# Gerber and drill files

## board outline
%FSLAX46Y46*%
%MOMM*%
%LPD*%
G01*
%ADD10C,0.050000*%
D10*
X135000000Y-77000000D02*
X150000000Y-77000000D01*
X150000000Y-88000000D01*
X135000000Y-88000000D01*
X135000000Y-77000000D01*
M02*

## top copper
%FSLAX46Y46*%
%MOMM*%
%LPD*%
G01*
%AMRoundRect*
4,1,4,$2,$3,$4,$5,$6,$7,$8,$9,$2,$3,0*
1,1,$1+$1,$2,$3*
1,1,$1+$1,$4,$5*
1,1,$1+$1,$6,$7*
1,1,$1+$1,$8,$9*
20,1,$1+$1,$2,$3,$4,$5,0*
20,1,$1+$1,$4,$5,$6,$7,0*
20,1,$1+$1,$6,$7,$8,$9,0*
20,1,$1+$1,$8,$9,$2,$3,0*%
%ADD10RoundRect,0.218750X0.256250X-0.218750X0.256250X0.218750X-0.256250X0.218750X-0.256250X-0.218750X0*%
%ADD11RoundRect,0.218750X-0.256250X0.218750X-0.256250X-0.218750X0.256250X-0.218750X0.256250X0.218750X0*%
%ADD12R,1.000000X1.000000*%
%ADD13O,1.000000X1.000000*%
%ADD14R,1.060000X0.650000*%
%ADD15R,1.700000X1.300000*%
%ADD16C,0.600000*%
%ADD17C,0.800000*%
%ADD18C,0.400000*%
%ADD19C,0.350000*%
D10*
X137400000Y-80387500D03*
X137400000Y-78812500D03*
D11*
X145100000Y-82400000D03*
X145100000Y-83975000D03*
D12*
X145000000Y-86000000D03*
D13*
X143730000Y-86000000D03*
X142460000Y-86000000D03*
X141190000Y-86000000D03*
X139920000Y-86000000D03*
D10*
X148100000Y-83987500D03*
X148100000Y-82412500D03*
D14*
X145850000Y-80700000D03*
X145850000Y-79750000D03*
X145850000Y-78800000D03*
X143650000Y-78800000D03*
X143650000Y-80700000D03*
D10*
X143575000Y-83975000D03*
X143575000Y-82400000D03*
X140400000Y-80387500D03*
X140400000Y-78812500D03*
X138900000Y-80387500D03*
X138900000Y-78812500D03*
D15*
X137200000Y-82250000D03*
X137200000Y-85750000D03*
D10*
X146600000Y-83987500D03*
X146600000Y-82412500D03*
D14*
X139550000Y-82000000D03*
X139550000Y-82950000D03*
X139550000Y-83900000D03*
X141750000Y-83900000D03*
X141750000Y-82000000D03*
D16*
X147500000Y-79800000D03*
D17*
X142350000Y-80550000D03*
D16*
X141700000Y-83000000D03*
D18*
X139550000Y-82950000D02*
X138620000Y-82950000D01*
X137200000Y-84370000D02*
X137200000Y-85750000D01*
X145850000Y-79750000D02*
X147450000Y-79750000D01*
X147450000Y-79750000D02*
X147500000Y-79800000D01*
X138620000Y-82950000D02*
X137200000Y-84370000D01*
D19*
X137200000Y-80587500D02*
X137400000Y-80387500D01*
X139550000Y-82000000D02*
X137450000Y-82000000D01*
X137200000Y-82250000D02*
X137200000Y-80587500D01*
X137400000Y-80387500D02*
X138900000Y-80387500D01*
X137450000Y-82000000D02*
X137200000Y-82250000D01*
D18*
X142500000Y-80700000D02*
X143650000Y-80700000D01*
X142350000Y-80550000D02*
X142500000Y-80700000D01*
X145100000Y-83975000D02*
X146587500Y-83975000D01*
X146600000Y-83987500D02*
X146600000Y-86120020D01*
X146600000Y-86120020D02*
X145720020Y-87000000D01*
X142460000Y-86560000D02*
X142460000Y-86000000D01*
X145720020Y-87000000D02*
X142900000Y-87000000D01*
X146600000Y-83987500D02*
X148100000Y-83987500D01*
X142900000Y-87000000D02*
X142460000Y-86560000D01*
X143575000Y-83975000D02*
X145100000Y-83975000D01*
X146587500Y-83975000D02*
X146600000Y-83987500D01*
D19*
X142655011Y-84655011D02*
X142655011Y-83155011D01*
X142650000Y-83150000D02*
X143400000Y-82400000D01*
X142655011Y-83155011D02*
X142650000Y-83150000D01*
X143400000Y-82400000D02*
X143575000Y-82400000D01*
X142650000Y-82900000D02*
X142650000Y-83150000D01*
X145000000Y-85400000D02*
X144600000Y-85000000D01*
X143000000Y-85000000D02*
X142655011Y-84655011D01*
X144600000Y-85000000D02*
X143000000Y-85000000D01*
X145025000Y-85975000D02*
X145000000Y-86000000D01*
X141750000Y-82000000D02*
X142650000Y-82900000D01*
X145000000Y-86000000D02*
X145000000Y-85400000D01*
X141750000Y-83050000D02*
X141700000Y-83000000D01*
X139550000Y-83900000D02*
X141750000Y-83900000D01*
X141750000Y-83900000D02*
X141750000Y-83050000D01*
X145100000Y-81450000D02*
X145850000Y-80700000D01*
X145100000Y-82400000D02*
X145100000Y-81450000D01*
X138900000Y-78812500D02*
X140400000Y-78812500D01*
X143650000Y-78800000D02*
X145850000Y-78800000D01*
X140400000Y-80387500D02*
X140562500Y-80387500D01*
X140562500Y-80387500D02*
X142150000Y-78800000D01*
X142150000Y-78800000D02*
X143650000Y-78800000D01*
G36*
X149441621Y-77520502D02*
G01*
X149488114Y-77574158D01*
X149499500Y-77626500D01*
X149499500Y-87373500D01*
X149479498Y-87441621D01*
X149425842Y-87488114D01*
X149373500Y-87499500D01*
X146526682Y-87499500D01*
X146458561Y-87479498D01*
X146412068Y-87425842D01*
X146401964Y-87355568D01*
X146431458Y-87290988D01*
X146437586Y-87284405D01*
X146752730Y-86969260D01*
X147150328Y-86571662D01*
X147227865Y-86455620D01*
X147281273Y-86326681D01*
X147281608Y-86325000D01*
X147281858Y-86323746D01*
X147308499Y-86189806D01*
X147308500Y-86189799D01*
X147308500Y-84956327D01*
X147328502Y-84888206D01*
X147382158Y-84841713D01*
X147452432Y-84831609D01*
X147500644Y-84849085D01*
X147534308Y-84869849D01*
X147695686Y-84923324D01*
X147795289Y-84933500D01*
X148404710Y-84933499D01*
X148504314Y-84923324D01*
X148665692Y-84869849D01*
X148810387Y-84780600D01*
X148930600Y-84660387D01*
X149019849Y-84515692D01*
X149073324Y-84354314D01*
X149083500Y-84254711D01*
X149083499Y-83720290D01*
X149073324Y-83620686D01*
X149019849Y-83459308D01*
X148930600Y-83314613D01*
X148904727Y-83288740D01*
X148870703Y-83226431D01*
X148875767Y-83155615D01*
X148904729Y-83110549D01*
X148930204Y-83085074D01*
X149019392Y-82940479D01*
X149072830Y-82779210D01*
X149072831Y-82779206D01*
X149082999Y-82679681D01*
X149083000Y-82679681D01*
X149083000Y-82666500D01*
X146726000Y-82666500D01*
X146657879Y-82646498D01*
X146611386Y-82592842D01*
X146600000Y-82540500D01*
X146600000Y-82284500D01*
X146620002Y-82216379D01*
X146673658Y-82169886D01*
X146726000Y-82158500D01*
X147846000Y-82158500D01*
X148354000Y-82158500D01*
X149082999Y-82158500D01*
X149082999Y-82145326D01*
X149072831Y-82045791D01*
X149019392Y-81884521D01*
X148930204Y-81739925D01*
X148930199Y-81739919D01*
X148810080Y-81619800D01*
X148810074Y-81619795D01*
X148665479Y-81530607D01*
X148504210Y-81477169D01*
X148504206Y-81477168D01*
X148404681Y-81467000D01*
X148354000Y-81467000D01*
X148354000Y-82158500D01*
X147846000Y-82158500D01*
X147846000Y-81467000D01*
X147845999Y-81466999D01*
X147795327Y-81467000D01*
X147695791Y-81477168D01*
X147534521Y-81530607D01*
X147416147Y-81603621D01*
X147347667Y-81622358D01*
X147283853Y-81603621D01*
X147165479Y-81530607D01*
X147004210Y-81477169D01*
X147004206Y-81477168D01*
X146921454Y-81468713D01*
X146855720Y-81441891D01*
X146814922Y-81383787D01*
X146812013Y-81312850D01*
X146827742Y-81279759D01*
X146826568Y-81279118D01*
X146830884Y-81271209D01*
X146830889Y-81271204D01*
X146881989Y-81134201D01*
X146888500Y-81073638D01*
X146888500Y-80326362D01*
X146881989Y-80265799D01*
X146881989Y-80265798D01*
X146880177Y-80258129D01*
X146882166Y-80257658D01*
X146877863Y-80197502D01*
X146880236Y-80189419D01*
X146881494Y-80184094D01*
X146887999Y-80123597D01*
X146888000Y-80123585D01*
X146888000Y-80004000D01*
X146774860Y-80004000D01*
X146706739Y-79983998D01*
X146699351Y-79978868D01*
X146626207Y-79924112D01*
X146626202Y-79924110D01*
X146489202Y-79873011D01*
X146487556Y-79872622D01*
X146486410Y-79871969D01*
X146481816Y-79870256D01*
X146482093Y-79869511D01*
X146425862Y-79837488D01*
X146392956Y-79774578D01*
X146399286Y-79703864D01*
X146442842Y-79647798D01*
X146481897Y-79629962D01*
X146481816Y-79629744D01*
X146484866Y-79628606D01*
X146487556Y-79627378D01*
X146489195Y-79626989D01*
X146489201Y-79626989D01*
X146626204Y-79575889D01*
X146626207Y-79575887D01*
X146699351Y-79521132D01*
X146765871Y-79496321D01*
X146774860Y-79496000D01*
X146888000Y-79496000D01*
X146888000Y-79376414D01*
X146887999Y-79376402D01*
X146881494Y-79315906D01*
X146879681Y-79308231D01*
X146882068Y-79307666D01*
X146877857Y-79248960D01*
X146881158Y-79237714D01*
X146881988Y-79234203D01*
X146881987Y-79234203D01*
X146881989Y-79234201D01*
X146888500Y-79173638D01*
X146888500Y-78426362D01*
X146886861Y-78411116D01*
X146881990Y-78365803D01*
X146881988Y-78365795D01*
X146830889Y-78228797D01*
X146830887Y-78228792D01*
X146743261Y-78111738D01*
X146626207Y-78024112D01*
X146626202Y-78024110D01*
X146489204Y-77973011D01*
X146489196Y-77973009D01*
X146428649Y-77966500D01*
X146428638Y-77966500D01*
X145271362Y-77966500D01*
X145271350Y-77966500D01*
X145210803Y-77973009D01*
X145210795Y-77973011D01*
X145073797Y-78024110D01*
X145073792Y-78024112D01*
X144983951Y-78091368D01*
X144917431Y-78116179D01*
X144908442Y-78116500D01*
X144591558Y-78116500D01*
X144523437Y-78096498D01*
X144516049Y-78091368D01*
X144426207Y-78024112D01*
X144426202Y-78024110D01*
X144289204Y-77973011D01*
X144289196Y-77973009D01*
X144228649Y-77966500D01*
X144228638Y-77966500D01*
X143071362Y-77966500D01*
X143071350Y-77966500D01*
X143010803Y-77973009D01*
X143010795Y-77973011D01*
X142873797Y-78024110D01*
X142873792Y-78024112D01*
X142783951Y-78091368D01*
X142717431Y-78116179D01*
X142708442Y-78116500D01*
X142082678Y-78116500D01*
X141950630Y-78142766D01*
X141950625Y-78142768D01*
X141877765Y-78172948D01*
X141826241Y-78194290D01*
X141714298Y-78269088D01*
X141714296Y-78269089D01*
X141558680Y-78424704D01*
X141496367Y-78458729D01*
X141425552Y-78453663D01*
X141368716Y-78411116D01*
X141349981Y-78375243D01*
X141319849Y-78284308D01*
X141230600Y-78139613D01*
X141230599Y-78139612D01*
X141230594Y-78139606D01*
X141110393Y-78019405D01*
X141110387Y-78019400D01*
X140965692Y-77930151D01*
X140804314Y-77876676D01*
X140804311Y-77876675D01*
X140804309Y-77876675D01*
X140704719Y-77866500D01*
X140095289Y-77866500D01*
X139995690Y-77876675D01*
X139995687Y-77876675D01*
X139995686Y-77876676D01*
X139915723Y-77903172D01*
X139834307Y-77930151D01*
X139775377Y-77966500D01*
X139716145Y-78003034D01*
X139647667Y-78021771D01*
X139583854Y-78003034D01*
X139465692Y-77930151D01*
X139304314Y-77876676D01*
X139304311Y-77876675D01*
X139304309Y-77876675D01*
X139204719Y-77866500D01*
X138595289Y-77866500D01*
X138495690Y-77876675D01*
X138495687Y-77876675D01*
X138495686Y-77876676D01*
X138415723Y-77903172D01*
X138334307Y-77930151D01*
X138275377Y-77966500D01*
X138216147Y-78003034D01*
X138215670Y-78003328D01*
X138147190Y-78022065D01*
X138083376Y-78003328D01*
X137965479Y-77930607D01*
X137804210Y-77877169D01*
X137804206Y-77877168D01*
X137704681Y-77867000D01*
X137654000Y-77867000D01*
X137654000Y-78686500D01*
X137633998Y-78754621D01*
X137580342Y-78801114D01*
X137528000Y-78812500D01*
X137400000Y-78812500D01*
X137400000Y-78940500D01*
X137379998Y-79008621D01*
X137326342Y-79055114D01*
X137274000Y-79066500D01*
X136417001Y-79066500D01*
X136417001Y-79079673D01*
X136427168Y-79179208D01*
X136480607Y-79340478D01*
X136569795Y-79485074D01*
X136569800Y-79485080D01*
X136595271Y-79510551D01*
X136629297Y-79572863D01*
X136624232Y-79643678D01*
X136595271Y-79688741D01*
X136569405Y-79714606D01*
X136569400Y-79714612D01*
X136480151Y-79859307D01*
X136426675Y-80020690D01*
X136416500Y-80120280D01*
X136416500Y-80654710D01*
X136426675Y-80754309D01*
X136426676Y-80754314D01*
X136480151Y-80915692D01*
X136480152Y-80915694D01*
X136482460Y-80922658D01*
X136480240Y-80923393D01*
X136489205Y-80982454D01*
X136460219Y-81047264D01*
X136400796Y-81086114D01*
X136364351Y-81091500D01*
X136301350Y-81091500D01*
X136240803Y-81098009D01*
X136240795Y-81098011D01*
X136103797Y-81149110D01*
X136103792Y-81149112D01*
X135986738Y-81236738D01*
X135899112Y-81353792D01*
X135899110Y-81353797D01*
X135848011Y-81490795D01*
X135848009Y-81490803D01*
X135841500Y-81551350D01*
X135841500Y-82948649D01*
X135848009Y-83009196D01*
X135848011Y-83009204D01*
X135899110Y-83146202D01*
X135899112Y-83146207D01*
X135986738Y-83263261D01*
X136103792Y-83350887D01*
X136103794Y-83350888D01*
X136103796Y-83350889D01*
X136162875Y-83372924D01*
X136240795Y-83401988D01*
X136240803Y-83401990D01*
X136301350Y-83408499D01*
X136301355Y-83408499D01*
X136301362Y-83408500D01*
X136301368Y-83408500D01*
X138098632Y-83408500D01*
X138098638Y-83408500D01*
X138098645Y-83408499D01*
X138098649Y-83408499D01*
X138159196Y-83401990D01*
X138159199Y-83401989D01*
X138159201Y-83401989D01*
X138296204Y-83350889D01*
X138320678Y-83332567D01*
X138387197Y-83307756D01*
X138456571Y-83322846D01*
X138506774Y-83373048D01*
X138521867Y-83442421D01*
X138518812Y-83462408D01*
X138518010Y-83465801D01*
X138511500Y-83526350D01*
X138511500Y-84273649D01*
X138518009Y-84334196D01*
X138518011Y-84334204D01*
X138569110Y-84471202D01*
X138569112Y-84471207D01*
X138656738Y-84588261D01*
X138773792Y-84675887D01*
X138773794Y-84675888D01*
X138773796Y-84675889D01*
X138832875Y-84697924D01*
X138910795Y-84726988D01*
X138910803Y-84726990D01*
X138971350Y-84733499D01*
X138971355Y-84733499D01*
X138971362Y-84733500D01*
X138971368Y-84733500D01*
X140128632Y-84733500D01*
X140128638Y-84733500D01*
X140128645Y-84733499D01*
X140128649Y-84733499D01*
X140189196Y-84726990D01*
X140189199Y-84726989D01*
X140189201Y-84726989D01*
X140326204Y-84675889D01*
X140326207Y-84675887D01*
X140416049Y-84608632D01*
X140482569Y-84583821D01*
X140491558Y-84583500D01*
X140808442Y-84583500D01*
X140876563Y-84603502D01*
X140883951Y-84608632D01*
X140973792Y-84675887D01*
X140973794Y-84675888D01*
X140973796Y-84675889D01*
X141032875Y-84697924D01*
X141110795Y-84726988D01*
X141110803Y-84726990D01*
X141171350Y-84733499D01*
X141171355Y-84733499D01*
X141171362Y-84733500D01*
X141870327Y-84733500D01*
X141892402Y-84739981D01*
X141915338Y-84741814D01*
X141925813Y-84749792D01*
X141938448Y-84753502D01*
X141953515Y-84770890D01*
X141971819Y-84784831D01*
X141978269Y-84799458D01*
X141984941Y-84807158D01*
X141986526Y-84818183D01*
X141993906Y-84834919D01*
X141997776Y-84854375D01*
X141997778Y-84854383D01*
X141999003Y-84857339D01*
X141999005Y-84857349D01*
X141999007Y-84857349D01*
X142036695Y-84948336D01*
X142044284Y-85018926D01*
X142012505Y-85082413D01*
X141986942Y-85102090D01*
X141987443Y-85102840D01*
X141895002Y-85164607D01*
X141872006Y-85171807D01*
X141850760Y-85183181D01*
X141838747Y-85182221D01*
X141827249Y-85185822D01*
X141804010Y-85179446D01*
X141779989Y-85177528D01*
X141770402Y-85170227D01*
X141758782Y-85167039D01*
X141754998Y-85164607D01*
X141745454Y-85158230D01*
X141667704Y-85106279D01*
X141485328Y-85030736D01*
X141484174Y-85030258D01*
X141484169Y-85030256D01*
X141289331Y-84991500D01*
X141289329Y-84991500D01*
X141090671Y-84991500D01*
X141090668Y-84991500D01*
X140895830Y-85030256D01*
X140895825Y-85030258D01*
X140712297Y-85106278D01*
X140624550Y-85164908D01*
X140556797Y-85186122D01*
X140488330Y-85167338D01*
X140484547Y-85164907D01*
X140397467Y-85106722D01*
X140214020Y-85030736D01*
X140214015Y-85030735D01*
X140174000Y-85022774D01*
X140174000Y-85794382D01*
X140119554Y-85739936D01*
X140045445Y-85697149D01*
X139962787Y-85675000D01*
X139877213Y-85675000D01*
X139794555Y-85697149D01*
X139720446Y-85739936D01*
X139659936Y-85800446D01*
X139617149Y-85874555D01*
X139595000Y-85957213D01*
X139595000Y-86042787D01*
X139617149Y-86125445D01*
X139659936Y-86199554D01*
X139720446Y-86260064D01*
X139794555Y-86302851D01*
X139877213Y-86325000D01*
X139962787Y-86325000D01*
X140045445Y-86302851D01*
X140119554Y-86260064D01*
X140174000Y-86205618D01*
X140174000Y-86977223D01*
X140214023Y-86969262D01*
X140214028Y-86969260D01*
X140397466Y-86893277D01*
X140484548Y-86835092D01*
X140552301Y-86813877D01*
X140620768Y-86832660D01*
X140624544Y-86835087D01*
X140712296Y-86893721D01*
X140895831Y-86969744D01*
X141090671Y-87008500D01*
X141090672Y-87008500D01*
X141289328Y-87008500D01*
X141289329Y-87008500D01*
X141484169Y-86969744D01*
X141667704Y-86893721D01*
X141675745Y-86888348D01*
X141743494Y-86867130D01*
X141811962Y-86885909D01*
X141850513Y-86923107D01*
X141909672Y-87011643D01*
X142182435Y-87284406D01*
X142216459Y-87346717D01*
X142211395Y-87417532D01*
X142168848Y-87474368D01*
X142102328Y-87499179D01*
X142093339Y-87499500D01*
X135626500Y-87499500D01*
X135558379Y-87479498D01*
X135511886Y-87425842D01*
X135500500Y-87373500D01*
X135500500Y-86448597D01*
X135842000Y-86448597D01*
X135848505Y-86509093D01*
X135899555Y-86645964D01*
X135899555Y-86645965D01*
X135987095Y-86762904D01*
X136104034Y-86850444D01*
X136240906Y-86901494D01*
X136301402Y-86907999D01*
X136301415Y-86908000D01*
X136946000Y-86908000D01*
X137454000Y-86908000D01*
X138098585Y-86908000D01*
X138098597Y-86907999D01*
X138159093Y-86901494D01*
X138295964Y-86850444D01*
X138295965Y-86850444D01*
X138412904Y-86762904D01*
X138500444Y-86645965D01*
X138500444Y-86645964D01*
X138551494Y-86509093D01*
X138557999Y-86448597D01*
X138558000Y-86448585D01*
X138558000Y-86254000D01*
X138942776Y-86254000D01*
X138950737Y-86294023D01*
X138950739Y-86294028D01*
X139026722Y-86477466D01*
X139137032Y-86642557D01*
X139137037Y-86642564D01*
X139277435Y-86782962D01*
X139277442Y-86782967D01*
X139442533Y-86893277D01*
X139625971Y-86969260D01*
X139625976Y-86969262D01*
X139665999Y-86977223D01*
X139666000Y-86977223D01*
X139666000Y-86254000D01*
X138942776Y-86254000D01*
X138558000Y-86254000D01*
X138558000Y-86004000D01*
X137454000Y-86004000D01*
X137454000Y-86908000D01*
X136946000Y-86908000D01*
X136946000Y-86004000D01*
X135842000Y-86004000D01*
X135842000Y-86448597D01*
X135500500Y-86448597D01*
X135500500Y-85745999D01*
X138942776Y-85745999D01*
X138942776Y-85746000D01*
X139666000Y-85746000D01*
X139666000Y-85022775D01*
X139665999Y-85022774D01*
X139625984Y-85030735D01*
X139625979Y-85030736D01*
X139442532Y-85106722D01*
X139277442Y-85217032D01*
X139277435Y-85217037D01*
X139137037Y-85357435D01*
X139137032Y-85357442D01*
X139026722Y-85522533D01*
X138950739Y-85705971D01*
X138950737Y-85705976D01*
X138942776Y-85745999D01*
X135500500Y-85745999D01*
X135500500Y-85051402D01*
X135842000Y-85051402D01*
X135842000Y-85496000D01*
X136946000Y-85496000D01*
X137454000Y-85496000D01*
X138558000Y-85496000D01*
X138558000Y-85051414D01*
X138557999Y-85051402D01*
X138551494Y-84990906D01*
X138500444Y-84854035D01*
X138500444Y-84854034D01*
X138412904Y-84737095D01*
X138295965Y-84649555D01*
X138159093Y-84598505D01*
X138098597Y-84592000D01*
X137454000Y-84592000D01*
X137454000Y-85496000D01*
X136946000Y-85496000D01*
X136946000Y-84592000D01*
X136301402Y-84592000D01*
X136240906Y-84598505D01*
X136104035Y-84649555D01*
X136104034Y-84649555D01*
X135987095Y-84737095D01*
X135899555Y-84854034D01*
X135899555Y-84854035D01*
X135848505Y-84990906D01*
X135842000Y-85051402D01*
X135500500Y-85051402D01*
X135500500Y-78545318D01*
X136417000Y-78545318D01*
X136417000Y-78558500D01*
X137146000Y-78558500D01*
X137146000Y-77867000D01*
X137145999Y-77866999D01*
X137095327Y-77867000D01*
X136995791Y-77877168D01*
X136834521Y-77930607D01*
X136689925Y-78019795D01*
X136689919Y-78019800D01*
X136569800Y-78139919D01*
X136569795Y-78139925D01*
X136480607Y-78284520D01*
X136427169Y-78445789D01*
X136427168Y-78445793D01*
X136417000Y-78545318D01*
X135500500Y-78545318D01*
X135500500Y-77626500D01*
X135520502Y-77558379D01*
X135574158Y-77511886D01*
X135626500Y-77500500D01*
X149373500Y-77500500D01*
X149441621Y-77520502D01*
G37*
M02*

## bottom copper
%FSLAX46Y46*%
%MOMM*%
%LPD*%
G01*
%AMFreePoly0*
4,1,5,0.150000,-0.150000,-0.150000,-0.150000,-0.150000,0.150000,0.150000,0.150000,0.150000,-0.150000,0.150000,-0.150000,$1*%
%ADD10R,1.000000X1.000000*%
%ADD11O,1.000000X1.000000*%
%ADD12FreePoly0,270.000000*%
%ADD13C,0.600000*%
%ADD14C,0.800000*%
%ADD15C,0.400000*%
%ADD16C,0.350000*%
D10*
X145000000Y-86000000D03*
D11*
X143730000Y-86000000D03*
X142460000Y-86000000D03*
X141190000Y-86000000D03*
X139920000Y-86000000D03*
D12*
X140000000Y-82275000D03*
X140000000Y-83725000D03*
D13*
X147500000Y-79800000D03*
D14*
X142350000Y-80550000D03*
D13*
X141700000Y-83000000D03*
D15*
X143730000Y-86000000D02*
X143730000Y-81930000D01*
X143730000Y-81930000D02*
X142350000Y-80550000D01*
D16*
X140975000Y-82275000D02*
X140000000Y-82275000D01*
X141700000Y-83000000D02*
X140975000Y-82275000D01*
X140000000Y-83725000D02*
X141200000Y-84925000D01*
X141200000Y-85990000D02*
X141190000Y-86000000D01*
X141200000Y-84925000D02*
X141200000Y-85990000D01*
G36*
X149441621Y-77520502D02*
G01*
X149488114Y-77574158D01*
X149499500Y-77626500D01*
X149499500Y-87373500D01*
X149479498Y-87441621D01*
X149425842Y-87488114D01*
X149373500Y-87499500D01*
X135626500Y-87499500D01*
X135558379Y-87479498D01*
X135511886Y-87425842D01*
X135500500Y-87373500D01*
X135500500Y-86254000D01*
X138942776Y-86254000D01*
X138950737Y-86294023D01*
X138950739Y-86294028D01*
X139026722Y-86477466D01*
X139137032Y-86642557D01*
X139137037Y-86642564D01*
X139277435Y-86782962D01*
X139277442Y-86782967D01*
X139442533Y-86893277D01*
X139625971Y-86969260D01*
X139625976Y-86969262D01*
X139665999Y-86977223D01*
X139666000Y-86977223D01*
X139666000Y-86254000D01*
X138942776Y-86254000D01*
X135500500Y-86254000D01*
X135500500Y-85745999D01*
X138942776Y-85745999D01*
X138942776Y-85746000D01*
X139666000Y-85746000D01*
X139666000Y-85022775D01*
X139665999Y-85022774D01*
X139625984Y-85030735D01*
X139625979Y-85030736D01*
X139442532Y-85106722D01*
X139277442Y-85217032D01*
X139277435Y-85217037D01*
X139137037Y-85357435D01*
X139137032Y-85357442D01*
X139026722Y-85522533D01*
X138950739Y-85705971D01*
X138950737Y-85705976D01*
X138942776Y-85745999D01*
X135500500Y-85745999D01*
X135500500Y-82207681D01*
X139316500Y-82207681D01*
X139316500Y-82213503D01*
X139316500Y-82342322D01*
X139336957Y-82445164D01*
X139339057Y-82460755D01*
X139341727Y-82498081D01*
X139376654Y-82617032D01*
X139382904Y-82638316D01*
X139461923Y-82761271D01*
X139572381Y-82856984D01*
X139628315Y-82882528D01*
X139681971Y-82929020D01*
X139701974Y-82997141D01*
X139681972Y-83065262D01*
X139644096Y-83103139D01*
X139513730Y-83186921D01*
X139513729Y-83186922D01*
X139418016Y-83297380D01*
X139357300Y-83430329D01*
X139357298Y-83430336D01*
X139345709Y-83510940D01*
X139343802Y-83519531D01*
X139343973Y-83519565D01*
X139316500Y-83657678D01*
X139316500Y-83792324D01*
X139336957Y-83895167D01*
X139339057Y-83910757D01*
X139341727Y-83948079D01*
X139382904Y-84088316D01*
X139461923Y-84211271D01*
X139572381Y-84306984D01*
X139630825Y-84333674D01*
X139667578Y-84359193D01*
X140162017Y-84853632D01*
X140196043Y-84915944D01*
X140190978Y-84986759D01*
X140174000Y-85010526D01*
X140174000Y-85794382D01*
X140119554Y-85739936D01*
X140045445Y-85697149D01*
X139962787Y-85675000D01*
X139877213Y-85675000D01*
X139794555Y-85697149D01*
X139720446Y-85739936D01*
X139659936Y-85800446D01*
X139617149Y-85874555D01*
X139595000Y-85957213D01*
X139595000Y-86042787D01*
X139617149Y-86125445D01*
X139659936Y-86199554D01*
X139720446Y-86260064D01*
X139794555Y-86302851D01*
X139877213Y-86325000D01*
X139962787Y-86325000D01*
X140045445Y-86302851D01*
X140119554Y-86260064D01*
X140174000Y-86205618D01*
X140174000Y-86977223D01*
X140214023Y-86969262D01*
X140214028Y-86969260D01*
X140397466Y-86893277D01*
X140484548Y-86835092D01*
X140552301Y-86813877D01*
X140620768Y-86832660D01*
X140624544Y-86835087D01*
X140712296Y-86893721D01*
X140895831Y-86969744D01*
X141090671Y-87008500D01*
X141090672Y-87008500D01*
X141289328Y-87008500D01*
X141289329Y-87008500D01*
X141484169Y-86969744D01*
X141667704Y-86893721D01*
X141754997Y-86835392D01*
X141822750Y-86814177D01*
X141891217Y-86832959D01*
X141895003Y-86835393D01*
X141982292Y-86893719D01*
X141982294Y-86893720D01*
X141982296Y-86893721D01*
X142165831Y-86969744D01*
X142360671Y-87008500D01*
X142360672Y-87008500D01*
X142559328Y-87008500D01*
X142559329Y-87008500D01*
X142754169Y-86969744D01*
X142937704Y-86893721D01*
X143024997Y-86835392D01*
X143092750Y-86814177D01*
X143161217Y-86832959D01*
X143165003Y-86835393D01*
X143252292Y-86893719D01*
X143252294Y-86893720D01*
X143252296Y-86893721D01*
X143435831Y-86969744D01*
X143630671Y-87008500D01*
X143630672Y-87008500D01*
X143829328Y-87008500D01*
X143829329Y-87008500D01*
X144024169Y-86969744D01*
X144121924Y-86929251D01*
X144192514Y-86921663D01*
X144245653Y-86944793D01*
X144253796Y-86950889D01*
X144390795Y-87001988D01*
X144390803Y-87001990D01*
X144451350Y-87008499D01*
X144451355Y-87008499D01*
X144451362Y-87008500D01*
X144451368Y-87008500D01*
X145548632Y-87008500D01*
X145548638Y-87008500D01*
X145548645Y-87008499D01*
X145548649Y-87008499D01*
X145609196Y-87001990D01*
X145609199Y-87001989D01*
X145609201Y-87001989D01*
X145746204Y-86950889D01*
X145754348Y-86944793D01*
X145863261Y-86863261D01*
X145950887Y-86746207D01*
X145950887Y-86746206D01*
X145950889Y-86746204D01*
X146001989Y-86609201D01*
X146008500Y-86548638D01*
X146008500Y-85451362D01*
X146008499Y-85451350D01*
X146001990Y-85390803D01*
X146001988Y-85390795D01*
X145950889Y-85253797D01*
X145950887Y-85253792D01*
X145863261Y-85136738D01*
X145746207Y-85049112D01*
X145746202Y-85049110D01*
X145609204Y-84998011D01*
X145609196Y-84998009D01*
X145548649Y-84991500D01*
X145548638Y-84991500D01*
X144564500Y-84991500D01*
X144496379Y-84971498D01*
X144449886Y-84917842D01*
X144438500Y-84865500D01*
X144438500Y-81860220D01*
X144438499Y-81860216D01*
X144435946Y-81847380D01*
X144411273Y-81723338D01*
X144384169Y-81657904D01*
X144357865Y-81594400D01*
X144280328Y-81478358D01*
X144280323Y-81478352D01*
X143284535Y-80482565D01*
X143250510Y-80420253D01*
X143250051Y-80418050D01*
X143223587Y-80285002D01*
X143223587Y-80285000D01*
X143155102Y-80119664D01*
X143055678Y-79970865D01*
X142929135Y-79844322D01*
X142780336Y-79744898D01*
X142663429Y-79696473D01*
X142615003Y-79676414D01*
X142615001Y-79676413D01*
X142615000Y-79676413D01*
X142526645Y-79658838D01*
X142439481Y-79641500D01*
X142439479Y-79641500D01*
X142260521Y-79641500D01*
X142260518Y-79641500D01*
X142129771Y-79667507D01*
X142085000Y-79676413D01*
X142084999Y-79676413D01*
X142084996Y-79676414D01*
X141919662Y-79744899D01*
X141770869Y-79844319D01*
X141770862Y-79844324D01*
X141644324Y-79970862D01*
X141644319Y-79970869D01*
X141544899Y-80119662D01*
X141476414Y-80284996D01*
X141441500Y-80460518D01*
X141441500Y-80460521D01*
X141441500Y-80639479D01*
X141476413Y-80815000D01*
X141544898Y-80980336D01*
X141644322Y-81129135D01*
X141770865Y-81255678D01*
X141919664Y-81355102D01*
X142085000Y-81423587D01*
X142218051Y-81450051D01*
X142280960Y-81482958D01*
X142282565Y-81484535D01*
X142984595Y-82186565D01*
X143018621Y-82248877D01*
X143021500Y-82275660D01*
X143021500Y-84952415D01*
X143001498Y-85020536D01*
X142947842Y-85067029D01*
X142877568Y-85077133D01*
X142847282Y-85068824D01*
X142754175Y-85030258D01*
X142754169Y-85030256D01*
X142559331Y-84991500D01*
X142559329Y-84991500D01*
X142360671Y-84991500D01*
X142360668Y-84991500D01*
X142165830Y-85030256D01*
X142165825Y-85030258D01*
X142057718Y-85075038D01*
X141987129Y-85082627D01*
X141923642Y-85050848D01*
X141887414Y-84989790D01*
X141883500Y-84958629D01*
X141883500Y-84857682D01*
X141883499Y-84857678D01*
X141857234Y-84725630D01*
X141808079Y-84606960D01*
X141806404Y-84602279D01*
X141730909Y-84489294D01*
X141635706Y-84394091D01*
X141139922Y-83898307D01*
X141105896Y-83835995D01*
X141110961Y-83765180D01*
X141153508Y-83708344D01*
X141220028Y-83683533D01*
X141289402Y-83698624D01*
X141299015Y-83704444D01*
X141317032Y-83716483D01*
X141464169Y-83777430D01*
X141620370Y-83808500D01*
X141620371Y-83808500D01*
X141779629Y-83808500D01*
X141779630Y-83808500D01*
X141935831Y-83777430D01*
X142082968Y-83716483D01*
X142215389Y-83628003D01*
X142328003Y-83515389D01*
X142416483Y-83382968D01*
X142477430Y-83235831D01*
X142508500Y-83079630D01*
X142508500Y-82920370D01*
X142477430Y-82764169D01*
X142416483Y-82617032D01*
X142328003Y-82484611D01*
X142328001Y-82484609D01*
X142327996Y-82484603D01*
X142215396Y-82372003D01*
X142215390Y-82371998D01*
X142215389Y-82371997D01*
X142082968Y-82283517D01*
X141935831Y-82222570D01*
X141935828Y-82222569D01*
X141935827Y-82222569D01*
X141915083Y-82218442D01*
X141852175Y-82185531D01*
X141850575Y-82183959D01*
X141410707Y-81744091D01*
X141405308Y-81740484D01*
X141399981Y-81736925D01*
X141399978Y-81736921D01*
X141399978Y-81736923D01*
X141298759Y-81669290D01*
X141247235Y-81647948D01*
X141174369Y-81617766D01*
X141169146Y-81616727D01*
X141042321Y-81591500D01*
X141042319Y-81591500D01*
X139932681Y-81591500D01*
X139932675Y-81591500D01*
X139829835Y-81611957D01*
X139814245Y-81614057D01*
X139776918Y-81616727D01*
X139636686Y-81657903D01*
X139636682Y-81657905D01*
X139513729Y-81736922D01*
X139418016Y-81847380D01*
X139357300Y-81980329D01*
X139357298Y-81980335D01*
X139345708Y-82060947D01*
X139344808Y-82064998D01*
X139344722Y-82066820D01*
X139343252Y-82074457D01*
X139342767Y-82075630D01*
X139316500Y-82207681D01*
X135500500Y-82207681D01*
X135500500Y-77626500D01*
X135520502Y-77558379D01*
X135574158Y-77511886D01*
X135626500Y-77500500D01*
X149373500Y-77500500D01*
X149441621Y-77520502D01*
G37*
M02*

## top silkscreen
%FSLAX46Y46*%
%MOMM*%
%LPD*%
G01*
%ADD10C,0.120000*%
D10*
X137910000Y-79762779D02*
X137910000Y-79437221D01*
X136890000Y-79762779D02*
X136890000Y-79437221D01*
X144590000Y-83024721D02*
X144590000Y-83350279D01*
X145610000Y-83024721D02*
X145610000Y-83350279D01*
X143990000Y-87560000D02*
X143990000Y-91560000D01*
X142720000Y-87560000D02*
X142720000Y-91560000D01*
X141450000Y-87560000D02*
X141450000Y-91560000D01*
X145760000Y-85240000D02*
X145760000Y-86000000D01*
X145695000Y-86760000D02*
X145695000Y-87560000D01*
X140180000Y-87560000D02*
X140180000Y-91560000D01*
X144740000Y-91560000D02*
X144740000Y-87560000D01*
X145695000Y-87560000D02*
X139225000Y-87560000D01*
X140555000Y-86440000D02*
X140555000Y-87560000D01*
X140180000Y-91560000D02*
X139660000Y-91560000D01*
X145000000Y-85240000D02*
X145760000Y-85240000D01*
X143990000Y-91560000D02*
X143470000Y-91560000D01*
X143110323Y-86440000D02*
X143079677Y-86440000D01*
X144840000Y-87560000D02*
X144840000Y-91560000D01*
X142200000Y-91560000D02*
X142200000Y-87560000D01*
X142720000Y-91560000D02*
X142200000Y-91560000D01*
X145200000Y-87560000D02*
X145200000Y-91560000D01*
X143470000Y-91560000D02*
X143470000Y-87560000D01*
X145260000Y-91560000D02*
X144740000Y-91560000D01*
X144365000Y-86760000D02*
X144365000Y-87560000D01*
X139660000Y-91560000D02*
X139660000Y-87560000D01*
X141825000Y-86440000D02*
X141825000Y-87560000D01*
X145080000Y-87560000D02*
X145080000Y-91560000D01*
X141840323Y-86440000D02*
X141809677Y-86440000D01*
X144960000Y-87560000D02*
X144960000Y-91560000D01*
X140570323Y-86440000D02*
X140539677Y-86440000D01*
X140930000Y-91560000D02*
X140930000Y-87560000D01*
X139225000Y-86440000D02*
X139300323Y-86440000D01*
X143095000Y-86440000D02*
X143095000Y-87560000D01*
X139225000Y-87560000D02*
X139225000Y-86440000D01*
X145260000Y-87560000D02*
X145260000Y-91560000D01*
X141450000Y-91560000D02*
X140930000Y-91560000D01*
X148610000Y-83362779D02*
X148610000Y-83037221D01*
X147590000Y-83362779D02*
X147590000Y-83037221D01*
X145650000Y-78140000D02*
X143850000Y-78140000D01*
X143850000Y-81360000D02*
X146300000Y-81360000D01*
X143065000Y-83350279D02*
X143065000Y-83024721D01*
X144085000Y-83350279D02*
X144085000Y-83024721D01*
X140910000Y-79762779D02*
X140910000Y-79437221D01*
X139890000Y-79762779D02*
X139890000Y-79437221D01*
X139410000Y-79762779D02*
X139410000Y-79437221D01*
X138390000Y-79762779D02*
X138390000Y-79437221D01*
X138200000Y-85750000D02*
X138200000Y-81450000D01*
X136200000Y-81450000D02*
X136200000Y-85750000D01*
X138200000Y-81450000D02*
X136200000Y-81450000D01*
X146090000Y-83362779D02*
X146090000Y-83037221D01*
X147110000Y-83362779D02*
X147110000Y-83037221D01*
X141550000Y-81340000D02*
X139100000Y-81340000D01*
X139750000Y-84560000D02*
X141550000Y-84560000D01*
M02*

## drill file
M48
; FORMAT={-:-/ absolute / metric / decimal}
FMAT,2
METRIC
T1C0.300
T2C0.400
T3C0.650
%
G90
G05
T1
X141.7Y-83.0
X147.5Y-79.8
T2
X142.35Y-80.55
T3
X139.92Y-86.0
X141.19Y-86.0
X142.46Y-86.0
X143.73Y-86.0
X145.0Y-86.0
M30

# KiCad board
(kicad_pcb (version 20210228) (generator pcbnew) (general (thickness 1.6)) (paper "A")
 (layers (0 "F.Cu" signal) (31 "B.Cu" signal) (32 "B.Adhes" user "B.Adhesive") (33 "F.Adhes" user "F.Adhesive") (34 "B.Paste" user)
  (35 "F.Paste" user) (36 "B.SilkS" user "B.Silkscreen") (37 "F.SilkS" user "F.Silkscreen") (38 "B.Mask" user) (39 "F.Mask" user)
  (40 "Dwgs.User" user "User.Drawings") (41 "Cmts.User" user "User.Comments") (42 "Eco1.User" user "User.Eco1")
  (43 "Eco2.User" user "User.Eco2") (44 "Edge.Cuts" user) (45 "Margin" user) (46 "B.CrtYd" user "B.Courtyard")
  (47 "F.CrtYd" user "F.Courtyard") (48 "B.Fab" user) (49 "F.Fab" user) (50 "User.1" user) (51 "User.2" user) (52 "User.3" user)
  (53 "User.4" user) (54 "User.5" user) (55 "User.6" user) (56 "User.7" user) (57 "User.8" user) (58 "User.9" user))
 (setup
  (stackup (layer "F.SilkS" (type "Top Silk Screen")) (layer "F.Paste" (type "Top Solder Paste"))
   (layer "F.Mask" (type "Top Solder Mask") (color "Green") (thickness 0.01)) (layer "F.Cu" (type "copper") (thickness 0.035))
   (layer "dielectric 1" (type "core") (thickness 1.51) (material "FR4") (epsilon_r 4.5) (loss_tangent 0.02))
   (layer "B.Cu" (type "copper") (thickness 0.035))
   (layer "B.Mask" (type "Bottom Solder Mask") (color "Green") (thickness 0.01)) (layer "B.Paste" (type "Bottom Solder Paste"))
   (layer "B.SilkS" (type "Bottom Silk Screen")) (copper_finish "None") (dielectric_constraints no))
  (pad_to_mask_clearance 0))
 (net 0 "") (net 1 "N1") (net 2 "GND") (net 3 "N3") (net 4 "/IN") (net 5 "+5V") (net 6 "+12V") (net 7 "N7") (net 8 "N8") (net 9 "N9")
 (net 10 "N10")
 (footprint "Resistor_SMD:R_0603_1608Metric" (layer "F.Cu") (at 137.4 79.6 90)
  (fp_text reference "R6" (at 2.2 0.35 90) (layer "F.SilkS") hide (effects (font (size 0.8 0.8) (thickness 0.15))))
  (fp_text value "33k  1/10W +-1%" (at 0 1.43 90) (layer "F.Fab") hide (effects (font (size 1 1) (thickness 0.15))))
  (fp_line (start -0.162779 0.51) (end 0.162779 0.51) (layer "F.SilkS") (width 0.12))
  (fp_line (start -0.162779 -0.51) (end 0.162779 -0.51) (layer "F.SilkS") (width 0.12))
  (pad "1" smd roundrect (at -0.7875 0 90) (locked) (size 0.875 0.95) (layers "F.Cu" "F.Paste" "F.Mask") (roundrect_rratio 0.25)
   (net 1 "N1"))
  (pad "2" smd roundrect (at 0.7875 0 90) (locked) (size 0.875 0.95) (layers "F.Cu" "F.Paste" "F.Mask") (roundrect_rratio 0.25)
   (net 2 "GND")))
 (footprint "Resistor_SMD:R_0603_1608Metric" (layer "F.Cu") (at 145.1 83.1875 -90)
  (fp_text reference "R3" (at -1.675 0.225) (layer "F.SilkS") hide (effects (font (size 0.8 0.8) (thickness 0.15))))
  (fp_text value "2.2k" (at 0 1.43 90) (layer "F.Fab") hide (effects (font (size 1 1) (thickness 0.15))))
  (fp_line (start -0.162779 0.51) (end 0.162779 0.51) (layer "F.SilkS") (width 0.12))
  (fp_line (start -0.162779 -0.51) (end 0.162779 -0.51) (layer "F.SilkS") (width 0.12))
  (pad "1" smd roundrect (at -0.7875 0 270) (locked) (size 0.875 0.95) (layers "F.Cu" "F.Paste" "F.Mask") (roundrect_rratio 0.25)
   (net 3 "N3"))
  (pad "2" smd roundrect (at 0.7875 0 270) (locked) (size 0.875 0.95) (layers "F.Cu" "F.Paste" "F.Mask") (roundrect_rratio 0.25)
   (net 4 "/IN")))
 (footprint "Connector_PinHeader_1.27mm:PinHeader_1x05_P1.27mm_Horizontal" (layer "F.Cu") (at 145 86 -90)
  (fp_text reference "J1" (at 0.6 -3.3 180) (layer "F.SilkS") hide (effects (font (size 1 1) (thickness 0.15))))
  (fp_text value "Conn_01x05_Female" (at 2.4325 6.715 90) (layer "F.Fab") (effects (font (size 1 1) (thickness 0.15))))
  (fp_line (start 1.56 1.01) (end 5.56 1.01) (layer "F.SilkS") (width 0.12))
  (fp_line (start 1.56 2.28) (end 5.56 2.28) (layer "F.SilkS") (width 0.12))
  (fp_line (start 1.56 3.55) (end 5.56 3.55) (layer "F.SilkS") (width 0.12))
  (fp_line (start -0.76 -0.76) (end 0 -0.76) (layer "F.SilkS") (width 0.12))
  (fp_line (start 0.76 -0.695) (end 1.56 -0.695) (layer "F.SilkS") (width 0.12))
  (fp_line (start 1.56 4.82) (end 5.56 4.82) (layer "F.SilkS") (width 0.12))
  (fp_line (start 5.56 0.26) (end 1.56 0.26) (layer "F.SilkS") (width 0.12))
  (fp_line (start 1.56 -0.695) (end 1.56 5.775) (layer "F.SilkS") (width 0.12))
  (fp_line (start 0.44 4.445) (end 1.56 4.445) (layer "F.SilkS") (width 0.12))
  (fp_line (start 5.56 4.82) (end 5.56 5.34) (layer "F.SilkS") (width 0.12))
  (fp_line (start -0.76 0) (end -0.76 -0.76) (layer "F.SilkS") (width 0.12))
  (fp_line (start 5.56 1.01) (end 5.56 1.53) (layer "F.SilkS") (width 0.12))
  (fp_line (start 0.44 1.889677) (end 0.44 1.920323) (layer "F.SilkS") (width 0.12))
  (fp_line (start 1.56 0.16) (end 5.56 0.16) (layer "F.SilkS") (width 0.12))
  (fp_line (start 5.56 2.8) (end 1.56 2.8) (layer "F.SilkS") (width 0.12))
  (fp_line (start 5.56 2.28) (end 5.56 2.8) (layer "F.SilkS") (width 0.12))
  (fp_line (start 1.56 -0.2) (end 5.56 -0.2) (layer "F.SilkS") (width 0.12))
  (fp_line (start 5.56 1.53) (end 1.56 1.53) (layer "F.SilkS") (width 0.12))
  (fp_line (start 5.56 -0.26) (end 5.56 0.26) (layer "F.SilkS") (width 0.12))
  (fp_line (start 0.76 0.635) (end 1.56 0.635) (layer "F.SilkS") (width 0.12))
  (fp_line (start 5.56 5.34) (end 1.56 5.34) (layer "F.SilkS") (width 0.12))
  (fp_line (start 0.44 3.175) (end 1.56 3.175) (layer "F.SilkS") (width 0.12))
  (fp_line (start 1.56 -0.08) (end 5.56 -0.08) (layer "F.SilkS") (width 0.12))
  (fp_line (start 0.44 3.159677) (end 0.44 3.190323) (layer "F.SilkS") (width 0.12))
  (fp_line (start 1.56 0.04) (end 5.56 0.04) (layer "F.SilkS") (width 0.12))
  (fp_line (start 0.44 4.429677) (end 0.44 4.460323) (layer "F.SilkS") (width 0.12))
  (fp_line (start 5.56 4.07) (end 1.56 4.07) (layer "F.SilkS") (width 0.12))
  (fp_line (start 0.44 5.775) (end 0.44 5.699677) (layer "F.SilkS") (width 0.12))
  (fp_line (start 0.44 1.905) (end 1.56 1.905) (layer "F.SilkS") (width 0.12))
  (fp_line (start 1.56 5.775) (end 0.44 5.775) (layer "F.SilkS") (width 0.12))
  (fp_line (start 1.56 -0.26) (end 5.56 -0.26) (layer "F.SilkS") (width 0.12))
  (fp_line (start 5.56 3.55) (end 5.56 4.07) (layer "F.SilkS") (width 0.12))
  (pad "1" thru_hole rect (at 0 0 270) (locked) (size 1 1) (drill 0.65) (layers *.Cu *.Mask) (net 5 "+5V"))
  (pad "2" thru_hole oval (at 0 1.27 270) (locked) (size 1 1) (drill 0.65) (layers *.Cu *.Mask) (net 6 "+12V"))
  (pad "3" thru_hole oval (at 0 2.54 270) (locked) (size 1 1) (drill 0.65) (layers *.Cu *.Mask) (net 4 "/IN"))
  (pad "4" thru_hole oval (at 0 3.81 270) (locked) (size 1 1) (drill 0.65) (layers *.Cu *.Mask) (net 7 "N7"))
  (pad "5" thru_hole oval (at 0 5.08 270) (locked) (size 1 1) (drill 0.65) (layers *.Cu *.Mask) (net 2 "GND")))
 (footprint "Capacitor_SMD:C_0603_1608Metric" (layer "F.Cu") (at 148.1 83.2 90)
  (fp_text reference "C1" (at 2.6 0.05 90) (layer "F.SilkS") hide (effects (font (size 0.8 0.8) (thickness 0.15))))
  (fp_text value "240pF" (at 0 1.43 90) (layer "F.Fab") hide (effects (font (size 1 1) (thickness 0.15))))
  (fp_line (start -0.162779 0.51) (end 0.162779 0.51) (layer "F.SilkS") (width 0.12))
  (fp_line (start -0.162779 -0.51) (end 0.162779 -0.51) (layer "F.SilkS") (width 0.12))
  (pad "1" smd roundrect (at -0.7875 0 90) (locked) (size 0.875 0.95) (layers "F.Cu" "F.Paste" "F.Mask") (roundrect_rratio 0.25)
   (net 4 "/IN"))
  (pad "2" smd roundrect (at 0.7875 0 90) (locked) (size 0.875 0.95) (layers "F.Cu" "F.Paste" "F.Mask") (roundrect_rratio 0.25)
   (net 2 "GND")))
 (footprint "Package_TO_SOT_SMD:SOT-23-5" (layer "F.Cu") (at 144.75 79.75 180)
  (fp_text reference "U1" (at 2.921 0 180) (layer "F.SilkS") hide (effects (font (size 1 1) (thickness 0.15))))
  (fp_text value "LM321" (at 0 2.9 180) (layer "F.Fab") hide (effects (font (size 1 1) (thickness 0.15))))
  (fp_line (start -0.9 1.61) (end 0.9 1.61) (layer "F.SilkS") (width 0.12))
  (fp_line (start 0.9 -1.61) (end -1.55 -1.61) (layer "F.SilkS") (width 0.12))
  (pad "1" smd rect (at -1.1 -0.95 180) (locked) (size 1.06 0.65) (layers "F.Cu" "F.Paste" "F.Mask") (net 3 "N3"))
  (pad "2" smd rect (at -1.1 0 180) (locked) (size 1.06 0.65) (layers "F.Cu" "F.Paste" "F.Mask") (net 2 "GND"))
  (pad "3" smd rect (at -1.1 0.95 180) (locked) (size 1.06 0.65) (layers "F.Cu" "F.Paste" "F.Mask") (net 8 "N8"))
  (pad "4" smd rect (at 1.1 0.95 180) (locked) (size 1.06 0.65) (layers "F.Cu" "F.Paste" "F.Mask") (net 8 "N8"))
  (pad "5" smd rect (at 1.1 -0.95 180) (locked) (size 1.06 0.65) (layers "F.Cu" "F.Paste" "F.Mask") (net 6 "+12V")))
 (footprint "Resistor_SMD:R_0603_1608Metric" (layer "F.Cu") (at 143.575 83.1875 90)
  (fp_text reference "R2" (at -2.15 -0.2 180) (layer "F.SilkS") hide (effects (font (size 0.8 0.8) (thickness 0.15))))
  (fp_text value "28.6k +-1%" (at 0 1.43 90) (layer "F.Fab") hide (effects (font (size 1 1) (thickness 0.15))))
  (fp_line (start -0.162779 -0.51) (end 0.162779 -0.51) (layer "F.SilkS") (width 0.12))
  (fp_line (start -0.162779 0.51) (end 0.162779 0.51) (layer "F.SilkS") (width 0.12))
  (pad "1" smd roundrect (at -0.7875 0 90) (locked) (size 0.875 0.95) (layers "F.Cu" "F.Paste" "F.Mask") (roundrect_rratio 0.25)
   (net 4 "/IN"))
  (pad "2" smd roundrect (at 0.7875 0 90) (locked) (size 0.875 0.95) (layers "F.Cu" "F.Paste" "F.Mask") (roundrect_rratio 0.25)
   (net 5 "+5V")))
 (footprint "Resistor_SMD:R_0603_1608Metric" (layer "F.Cu") (at 140.4 79.6 90)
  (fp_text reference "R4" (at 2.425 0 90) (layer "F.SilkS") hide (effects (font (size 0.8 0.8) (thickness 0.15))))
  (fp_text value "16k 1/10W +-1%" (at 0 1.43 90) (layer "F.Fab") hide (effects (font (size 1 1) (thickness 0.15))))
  (fp_line (start -0.162779 0.51) (end 0.162779 0.51) (layer "F.SilkS") (width 0.12))
  (fp_line (start -0.162779 -0.51) (end 0.162779 -0.51) (layer "F.SilkS") (width 0.12))
  (pad "1" smd roundrect (at -0.7875 0 90) (locked) (size 0.875 0.95) (layers "F.Cu" "F.Paste" "F.Mask") (roundrect_rratio 0.25)
   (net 8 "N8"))
  (pad "2" smd roundrect (at 0.7875 0 90) (locked) (size 0.875 0.95) (layers "F.Cu" "F.Paste" "F.Mask") (roundrect_rratio 0.25) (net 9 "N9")))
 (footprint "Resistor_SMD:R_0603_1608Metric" (layer "F.Cu") (at 138.9 79.6 90)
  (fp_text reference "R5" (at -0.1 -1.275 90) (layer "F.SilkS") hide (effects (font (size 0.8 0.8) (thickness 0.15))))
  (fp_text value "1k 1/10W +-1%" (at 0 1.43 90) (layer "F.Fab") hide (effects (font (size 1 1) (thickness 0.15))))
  (fp_line (start -0.162779 0.51) (end 0.162779 0.51) (layer "F.SilkS") (width 0.12))
  (fp_line (start -0.162779 -0.51) (end 0.162779 -0.51) (layer "F.SilkS") (width 0.12))
  (pad "1" smd roundrect (at -0.7875 0 90) (locked) (size 0.875 0.95) (layers "F.Cu" "F.Paste" "F.Mask") (roundrect_rratio 0.25)
   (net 1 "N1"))
  (pad "2" smd roundrect (at 0.7875 0 90) (locked) (size 0.875 0.95) (layers "F.Cu" "F.Paste" "F.Mask") (roundrect_rratio 0.25) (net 9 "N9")))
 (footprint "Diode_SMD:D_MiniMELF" (layer "F.Cu") (at 137.2 84 -90)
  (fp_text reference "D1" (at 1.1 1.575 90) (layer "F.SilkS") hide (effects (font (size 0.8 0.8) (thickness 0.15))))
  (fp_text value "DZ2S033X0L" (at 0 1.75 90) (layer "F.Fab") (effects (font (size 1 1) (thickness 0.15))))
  (fp_line (start 1.75 -1) (end -2.55 -1) (layer "F.SilkS") (width 0.12))
  (fp_line (start -2.55 1) (end 1.75 1) (layer "F.SilkS") (width 0.12))
  (fp_line (start -2.55 -1) (end -2.55 1) (layer "F.SilkS") (width 0.12))
  (pad "1" smd rect (at -1.75 0 270) (locked) (size 1.3 1.7) (layers "F.Cu" "F.Paste" "F.Mask") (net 1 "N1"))
  (pad "2" smd rect (at 1.75 0 270) (locked) (size 1.3 1.7) (layers "F.Cu" "F.Paste" "F.Mask") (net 2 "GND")))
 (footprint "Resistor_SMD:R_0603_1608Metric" (layer "F.Cu") (at 146.6 83.2 90)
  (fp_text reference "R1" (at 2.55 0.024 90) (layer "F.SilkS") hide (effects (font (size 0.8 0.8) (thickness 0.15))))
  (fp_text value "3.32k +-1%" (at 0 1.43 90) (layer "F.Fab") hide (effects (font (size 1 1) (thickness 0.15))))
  (fp_line (start -0.162779 -0.51) (end 0.162779 -0.51) (layer "F.SilkS") (width 0.12))
  (fp_line (start -0.162779 0.51) (end 0.162779 0.51) (layer "F.SilkS") (width 0.12))
  (pad "1" smd roundrect (at -0.7875 0 90) (locked) (size 0.875 0.95) (layers "F.Cu" "F.Paste" "F.Mask") (roundrect_rratio 0.25)
   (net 4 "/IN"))
  (pad "2" smd roundrect (at 0.7875 0 90) (locked) (size 0.875 0.95) (layers "F.Cu" "F.Paste" "F.Mask") (roundrect_rratio 0.25)
   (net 2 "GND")))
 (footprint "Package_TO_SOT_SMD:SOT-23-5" (layer "F.Cu") (at 140.65 82.95)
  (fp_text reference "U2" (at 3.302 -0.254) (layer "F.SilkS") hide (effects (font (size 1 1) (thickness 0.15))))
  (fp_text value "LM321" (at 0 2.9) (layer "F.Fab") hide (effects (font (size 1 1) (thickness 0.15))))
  (fp_line (start 0.9 -1.61) (end -1.55 -1.61) (layer "F.SilkS") (width 0.12))
  (fp_line (start -0.9 1.61) (end 0.9 1.61) (layer "F.SilkS") (width 0.12))
  (pad "1" smd rect (at -1.1 -0.95) (locked) (size 1.06 0.65) (layers "F.Cu" "F.Paste" "F.Mask") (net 1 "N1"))
  (pad "2" smd rect (at -1.1 0) (locked) (size 1.06 0.65) (layers "F.Cu" "F.Paste" "F.Mask") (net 2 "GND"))
  (pad "3" smd rect (at -1.1 0.95) (locked) (size 1.06 0.65) (layers "F.Cu" "F.Paste" "F.Mask") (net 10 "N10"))
  (pad "4" smd rect (at 1.1 0.95) (locked) (size 1.06 0.65) (layers "F.Cu" "F.Paste" "F.Mask") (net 10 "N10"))
  (pad "5" smd rect (at 1.1 -0.95) (locked) (size 1.06 0.65) (layers "F.Cu" "F.Paste" "F.Mask") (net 5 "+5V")))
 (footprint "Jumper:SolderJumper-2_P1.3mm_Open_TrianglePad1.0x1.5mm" (layer "B.Cu") (at 140 83 -90)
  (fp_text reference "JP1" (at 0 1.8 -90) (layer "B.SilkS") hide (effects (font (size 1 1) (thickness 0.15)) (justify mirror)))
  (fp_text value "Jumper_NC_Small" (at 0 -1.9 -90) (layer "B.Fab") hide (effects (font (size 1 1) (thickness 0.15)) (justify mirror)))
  (pad "1" smd custom (at -0.725 0 270) (locked) (size 0.3 0.3) (layers "B.Cu" "B.Mask") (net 10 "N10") (zone_connect 2)
   (options (clearance outline) (anchor rect)) (primitives))
  (pad "2" smd custom (at 0.725 0 270) (locked) (size 0.3 0.3) (layers "B.Cu" "B.Mask") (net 7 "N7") (zone_connect 2)
   (options (clearance outline) (anchor rect)) (primitives)))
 (gr_rect (start 150 77) (end 135 88) (layer "Edge.Cuts") (width 0.05) (fill none))
 (segment (start 139.55 82.95) (end 138.62 82.95) (width 0.4) (layer "F.Cu") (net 2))
 (segment (start 137.2 84.37) (end 137.2 85.75) (width 0.4) (layer "F.Cu") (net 2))
 (segment (start 145.85 79.75) (end 147.45 79.75) (width 0.4) (layer "F.Cu") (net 2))
 (segment (start 147.45 79.75) (end 147.5 79.8) (width 0.4) (layer "F.Cu") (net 2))
 (segment (start 138.62 82.95) (end 137.2 84.37) (width 0.4) (layer "F.Cu") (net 2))
 (via (at 147.5 79.8) (size 0.6) (drill 0.3) (layers "F.Cu" "B.Cu") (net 2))
 (segment (start 137.2 80.5875) (end 137.4 80.3875) (width 0.35) (layer "F.Cu") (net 1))
 (segment (start 139.55 82) (end 137.45 82) (width 0.35) (layer "F.Cu") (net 1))
 (segment (start 137.2 82.25) (end 137.2 80.5875) (width 0.35) (layer "F.Cu") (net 1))
 (segment (start 137.4 80.3875) (end 138.9 80.3875) (width 0.35) (layer "F.Cu") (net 1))
 (segment (start 137.45 82) (end 137.2 82.25) (width 0.35) (layer "F.Cu") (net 1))
 (segment (start 142.5 80.7) (end 143.65 80.7) (width 0.4) (layer "F.Cu") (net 6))
 (segment (start 142.35 80.55) (end 142.5 80.7) (width 0.4) (layer "F.Cu") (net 6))
 (via (at 142.35 80.55) (size 0.8) (drill 0.4) (layers "F.Cu" "B.Cu") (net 6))
 (segment (start 143.73 86) (end 143.73 81.93) (width 0.4) (layer "B.Cu") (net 6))
 (segment (start 143.73 81.93) (end 142.35 80.55) (width 0.4) (layer "B.Cu") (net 6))
 (segment (start 145.1 83.975) (end 146.5875 83.975) (width 0.4) (layer "F.Cu") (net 4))
 (segment (start 146.6 83.9875) (end 146.6 86.12002) (width 0.4) (layer "F.Cu") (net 4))
 (segment (start 146.6 86.12002) (end 145.72002 87) (width 0.4) (layer "F.Cu") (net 4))
 (segment (start 142.46 86.56) (end 142.46 86) (width 0.4) (layer "F.Cu") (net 4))
 (segment (start 145.72002 87) (end 142.9 87) (width 0.4) (layer "F.Cu") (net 4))
 (segment (start 146.6 83.9875) (end 148.1 83.9875) (width 0.4) (layer "F.Cu") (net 4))
 (segment (start 142.9 87) (end 142.46 86.56) (width 0.4) (layer "F.Cu") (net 4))
 (segment (start 143.575 83.975) (end 145.1 83.975) (width 0.4) (layer "F.Cu") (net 4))
 (segment (start 146.5875 83.975) (end 146.6 83.9875) (width 0.4) (layer "F.Cu") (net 4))
 (segment (start 142.655011 84.655011) (end 142.655011 83.155011) (width 0.35) (layer "F.Cu") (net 5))
 (segment (start 142.65 83.15) (end 143.4 82.4) (width 0.35) (layer "F.Cu") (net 5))
 (segment (start 142.655011 83.155011) (end 142.65 83.15) (width 0.35) (layer "F.Cu") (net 5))
 (segment (start 143.4 82.4) (end 143.575 82.4) (width 0.35) (layer "F.Cu") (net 5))
 (segment (start 142.65 82.9) (end 142.65 83.15) (width 0.35) (layer "F.Cu") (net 5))
 (segment (start 145 85.4) (end 144.6 85) (width 0.35) (layer "F.Cu") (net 5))
 (segment (start 143 85) (end 142.655011 84.655011) (width 0.35) (layer "F.Cu") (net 5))
 (segment (start 144.6 85) (end 143 85) (width 0.35) (layer "F.Cu") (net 5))
 (segment (start 145.025 85.975) (end 145 86) (width 0.35) (layer "F.Cu") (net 5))
 (segment (start 141.75 82) (end 142.65 82.9) (width 0.35) (layer "F.Cu") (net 5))
 (segment (start 145 86) (end 145 85.4) (width 0.35) (layer "F.Cu") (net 5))
 (segment (start 141.75 83.05) (end 141.7 83) (width 0.35) (layer "F.Cu") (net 10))
 (segment (start 139.55 83.9) (end 141.75 83.9) (width 0.35) (layer "F.Cu") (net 10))
 (segment (start 141.75 83.9) (end 141.75 83.05) (width 0.35) (layer "F.Cu") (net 10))
 (via (at 141.7 83) (size 0.6) (drill 0.3) (layers "F.Cu" "B.Cu") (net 10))
 (segment (start 140.975 82.275) (end 140 82.275) (width 0.35) (layer "B.Cu") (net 10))
 (segment (start 141.7 83) (end 140.975 82.275) (width 0.35) (layer "B.Cu") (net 10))
 (segment (start 145.1 81.45) (end 145.85 80.7) (width 0.35) (layer "F.Cu") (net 3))
 (segment (start 145.1 82.4) (end 145.1 81.45) (width 0.35) (layer "F.Cu") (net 3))
 (segment (start 138.9 78.8125) (end 140.4 78.8125) (width 0.35) (layer "F.Cu") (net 9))
 (segment (start 143.65 78.8) (end 145.85 78.8) (width 0.35) (layer "F.Cu") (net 8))
 (segment (start 140.4 80.3875) (end 140.5625 80.3875) (width 0.35) (layer "F.Cu") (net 8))
 (segment (start 140.5625 80.3875) (end 142.15 78.8) (width 0.35) (layer "F.Cu") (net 8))
 (segment (start 142.15 78.8) (end 143.65 78.8) (width 0.35) (layer "F.Cu") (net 8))
 (segment (start 140 83.725) (end 141.2 84.925) (width 0.35) (layer "B.Cu") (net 7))
 (segment (start 141.2 85.99) (end 141.19 86) (width 0.35) (layer "B.Cu") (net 7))
 (segment (start 141.2 84.925) (end 141.2 85.99) (width 0.35) (layer "B.Cu") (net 7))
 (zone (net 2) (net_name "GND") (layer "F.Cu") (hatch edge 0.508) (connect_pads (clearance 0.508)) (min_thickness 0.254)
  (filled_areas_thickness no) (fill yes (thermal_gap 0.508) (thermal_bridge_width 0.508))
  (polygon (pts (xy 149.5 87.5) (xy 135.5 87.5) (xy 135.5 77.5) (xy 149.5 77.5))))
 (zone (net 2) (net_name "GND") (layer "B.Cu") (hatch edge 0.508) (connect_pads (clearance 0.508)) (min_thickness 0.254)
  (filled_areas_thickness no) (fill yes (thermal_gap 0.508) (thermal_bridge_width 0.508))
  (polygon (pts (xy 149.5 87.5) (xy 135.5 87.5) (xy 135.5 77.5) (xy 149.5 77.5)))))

